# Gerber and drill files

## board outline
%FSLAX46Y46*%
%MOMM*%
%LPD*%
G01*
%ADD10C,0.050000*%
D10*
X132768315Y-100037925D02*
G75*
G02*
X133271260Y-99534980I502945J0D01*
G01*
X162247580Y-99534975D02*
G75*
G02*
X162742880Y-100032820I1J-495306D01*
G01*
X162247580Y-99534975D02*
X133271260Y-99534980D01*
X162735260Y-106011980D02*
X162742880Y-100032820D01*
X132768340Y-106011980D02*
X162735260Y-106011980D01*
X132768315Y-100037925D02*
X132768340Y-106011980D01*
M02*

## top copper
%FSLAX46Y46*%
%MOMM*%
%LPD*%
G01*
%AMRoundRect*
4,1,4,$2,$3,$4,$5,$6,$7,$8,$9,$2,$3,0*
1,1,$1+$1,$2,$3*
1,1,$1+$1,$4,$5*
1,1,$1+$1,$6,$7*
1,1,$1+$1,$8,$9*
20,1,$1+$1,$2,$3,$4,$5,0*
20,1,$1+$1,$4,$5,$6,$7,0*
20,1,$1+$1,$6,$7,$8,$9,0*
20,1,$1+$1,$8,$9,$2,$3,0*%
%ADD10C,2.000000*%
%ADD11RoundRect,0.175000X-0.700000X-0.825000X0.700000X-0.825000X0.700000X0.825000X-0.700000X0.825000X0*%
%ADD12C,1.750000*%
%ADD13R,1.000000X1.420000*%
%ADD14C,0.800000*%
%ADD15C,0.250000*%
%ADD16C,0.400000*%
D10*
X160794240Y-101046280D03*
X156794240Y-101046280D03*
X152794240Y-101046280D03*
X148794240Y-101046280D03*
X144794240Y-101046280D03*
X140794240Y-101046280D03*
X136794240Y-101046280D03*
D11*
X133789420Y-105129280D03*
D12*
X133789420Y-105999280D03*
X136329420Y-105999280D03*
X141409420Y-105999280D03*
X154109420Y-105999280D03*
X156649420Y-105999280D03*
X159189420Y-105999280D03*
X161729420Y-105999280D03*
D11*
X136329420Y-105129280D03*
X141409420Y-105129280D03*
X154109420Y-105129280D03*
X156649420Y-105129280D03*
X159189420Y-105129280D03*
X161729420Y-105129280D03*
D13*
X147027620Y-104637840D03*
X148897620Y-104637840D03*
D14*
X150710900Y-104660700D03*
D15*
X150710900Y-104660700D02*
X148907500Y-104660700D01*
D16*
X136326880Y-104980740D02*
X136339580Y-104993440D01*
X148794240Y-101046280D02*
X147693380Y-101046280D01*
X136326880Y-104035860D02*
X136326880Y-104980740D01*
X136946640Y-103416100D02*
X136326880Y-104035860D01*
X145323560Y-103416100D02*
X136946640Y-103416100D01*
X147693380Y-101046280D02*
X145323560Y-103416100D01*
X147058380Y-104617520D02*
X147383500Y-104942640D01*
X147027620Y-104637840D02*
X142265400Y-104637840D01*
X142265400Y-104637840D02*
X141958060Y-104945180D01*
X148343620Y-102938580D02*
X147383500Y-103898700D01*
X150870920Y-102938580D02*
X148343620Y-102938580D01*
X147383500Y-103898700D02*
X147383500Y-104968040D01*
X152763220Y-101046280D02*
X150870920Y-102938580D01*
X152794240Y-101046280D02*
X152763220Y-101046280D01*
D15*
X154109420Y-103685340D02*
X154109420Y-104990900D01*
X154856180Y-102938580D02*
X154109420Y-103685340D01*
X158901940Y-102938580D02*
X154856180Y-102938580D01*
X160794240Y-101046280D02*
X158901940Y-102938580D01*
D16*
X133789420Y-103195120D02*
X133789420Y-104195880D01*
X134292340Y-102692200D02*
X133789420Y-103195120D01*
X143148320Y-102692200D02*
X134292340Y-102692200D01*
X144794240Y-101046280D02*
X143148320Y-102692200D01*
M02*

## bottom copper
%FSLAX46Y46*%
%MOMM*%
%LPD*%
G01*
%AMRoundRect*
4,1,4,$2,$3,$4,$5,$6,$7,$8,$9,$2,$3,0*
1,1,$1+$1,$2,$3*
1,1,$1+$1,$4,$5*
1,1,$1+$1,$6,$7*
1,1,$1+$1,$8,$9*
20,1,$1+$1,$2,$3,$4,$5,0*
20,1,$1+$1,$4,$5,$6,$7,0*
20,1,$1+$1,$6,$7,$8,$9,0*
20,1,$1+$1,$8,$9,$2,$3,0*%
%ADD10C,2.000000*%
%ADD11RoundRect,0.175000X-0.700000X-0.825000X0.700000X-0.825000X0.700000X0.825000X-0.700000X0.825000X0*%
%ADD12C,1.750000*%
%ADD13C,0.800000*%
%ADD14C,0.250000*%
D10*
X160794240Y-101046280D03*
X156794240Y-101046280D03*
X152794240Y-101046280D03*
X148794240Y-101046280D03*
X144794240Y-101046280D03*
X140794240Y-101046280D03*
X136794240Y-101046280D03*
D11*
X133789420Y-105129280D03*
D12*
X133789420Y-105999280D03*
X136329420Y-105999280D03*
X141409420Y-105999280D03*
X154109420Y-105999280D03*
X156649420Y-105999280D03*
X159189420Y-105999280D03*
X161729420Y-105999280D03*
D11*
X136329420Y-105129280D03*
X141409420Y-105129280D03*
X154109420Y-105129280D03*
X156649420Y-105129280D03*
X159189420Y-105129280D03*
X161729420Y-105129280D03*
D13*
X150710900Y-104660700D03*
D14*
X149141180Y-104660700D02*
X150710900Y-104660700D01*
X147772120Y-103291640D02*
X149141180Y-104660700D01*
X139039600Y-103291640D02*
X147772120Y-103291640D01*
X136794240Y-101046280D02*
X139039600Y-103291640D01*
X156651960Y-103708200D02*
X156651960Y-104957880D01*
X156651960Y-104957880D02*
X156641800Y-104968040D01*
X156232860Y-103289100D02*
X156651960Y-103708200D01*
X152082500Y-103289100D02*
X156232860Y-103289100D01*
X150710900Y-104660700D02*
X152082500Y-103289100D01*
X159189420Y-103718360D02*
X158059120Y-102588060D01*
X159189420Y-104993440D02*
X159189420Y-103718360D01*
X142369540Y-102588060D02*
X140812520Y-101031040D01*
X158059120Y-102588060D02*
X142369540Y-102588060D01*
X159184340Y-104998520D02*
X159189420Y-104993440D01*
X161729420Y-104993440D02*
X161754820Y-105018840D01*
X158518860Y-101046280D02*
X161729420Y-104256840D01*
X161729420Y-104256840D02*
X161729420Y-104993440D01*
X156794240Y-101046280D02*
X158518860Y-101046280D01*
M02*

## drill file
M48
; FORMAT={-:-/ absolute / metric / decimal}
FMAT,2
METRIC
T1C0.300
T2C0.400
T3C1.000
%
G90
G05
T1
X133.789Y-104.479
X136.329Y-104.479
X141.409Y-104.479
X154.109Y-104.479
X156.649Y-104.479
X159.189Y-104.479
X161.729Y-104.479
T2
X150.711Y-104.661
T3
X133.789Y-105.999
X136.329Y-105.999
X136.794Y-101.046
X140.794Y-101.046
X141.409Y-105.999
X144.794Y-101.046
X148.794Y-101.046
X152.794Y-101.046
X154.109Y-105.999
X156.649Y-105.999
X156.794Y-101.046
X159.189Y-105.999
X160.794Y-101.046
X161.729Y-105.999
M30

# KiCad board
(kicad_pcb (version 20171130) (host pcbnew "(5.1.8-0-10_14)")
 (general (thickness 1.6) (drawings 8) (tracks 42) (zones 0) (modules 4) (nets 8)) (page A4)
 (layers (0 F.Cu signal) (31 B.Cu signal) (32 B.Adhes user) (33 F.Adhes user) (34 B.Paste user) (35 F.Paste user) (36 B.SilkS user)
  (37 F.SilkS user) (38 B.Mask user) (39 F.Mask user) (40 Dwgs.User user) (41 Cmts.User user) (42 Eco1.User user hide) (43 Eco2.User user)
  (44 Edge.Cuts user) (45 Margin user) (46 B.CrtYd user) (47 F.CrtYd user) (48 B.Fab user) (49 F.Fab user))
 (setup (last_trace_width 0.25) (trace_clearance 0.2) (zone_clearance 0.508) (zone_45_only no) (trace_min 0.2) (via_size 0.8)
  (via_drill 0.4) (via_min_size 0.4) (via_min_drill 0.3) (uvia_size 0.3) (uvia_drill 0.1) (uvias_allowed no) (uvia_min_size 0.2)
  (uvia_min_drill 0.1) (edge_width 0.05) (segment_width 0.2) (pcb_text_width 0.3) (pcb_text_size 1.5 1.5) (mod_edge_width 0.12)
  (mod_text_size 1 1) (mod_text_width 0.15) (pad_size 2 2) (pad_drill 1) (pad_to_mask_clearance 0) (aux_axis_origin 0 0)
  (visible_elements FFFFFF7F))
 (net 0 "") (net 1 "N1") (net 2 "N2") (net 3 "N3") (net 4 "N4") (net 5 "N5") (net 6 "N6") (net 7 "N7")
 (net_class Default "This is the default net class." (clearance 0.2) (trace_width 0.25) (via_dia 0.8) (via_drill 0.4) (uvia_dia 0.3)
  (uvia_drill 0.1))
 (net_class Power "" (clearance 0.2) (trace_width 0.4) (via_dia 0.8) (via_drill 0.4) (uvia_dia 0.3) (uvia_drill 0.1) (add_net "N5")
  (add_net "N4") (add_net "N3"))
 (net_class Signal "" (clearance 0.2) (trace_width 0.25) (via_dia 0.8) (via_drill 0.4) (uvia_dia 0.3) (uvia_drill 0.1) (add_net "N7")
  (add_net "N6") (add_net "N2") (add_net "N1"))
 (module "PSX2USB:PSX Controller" (layer F.Cu) (at 136.79424 101.04628)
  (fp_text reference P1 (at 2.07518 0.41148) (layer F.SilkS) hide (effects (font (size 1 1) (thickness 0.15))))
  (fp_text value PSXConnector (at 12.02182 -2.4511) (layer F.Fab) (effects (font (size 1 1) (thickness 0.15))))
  (pad 7 thru_hole circle (at 24 0) (size 2 2) (drill 1) (layers *.Cu *.Mask) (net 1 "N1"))
  (pad 6 thru_hole circle (at 20 0) (size 2 2) (drill 1) (layers *.Cu *.Mask) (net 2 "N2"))
  (pad 5 thru_hole circle (at 16 0) (size 2 2) (drill 1) (layers *.Cu *.Mask) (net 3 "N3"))
  (pad 4 thru_hole circle (at 12 0) (size 2 2) (drill 1) (layers *.Cu *.Mask) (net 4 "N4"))
  (pad 3 thru_hole circle (at 8 0) (size 2 2) (drill 1) (layers *.Cu *.Mask) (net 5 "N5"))
  (pad 2 thru_hole circle (at 4 0) (size 2 2) (drill 1) (layers *.Cu *.Mask) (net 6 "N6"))
  (pad 1 thru_hole circle (at 0 0) (size 2 2) (drill 1) (layers *.Cu *.Mask) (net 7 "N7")))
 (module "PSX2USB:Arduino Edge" (layer F.Cu) (at 136.32942 105.99928)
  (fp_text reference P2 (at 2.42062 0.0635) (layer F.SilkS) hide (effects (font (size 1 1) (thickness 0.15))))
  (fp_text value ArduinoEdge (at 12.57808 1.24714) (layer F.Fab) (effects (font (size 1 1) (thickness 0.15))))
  (pad 103 thru_hole roundrect (at -2.54 -1.52) (size 1.75 2) (drill 0.3 (offset 0 0.65)) (layers *.Cu *.Mask) (roundrect_rratio 0.1)
   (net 5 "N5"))
  (pad 103 thru_hole circle (at -2.54 0) (size 1.75 1.75) (drill 1) (layers *.Cu *.Mask) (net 5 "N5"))
  (pad 102 thru_hole circle (at 0 0) (size 1.75 1.75) (drill 1) (layers *.Cu *.Mask) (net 4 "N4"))
  (pad 101 thru_hole circle (at 5.08 0) (size 1.75 1.75) (drill 1) (layers *.Cu *.Mask) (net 3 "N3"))
  (pad 15 thru_hole circle (at 17.78 0) (size 1.75 1.75) (drill 1) (layers *.Cu *.Mask) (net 1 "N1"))
  (pad 14 thru_hole circle (at 20.32 0) (size 1.75 1.75) (drill 1) (layers *.Cu *.Mask) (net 7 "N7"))
  (pad 16 thru_hole circle (at 22.86 0) (size 1.75 1.75) (drill 1) (layers *.Cu *.Mask) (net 6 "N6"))
  (pad 10 thru_hole circle (at 25.4 0) (size 1.75 1.75) (drill 1) (layers *.Cu *.Mask) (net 2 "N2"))
  (pad 102 thru_hole roundrect (at 0 -1.52) (size 1.75 2) (drill 0.3 (offset 0 0.65)) (layers *.Cu *.Mask) (roundrect_rratio 0.1)
   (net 4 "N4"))
  (pad 101 thru_hole roundrect (at 5.08 -1.52) (size 1.75 2) (drill 0.3 (offset 0 0.65)) (layers *.Cu *.Mask) (roundrect_rratio 0.1)
   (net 3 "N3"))
  (pad 15 thru_hole roundrect (at 17.78 -1.52) (size 1.75 2) (drill 0.3 (offset 0 0.65)) (layers *.Cu *.Mask) (roundrect_rratio 0.1)
   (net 1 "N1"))
  (pad 14 thru_hole roundrect (at 20.32 -1.52) (size 1.75 2) (drill 0.3 (offset 0 0.65)) (layers *.Cu *.Mask) (roundrect_rratio 0.1)
   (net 7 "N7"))
  (pad 16 thru_hole roundrect (at 22.86 -1.52) (size 1.75 2) (drill 0.3 (offset 0 0.65)) (layers *.Cu *.Mask) (roundrect_rratio 0.1)
   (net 6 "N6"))
  (pad 10 thru_hole roundrect (at 25.4 -1.52) (size 1.75 2) (drill 0.3 (offset 0 0.65)) (layers *.Cu *.Mask) (roundrect_rratio 0.1)
   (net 2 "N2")))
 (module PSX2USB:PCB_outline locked (layer B.Cu) (at 162.74796 99.5299 180)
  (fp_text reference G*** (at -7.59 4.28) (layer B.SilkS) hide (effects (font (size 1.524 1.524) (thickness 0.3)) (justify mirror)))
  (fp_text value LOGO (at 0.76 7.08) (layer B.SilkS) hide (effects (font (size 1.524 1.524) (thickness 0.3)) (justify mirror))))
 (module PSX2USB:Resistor (layer F.Cu) (at 147.96262 104.63784 180)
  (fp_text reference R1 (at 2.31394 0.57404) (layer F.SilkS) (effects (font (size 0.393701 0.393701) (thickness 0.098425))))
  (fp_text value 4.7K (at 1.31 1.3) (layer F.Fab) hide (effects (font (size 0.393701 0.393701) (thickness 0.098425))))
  (pad 2 smd rect (at 0.935 0 180) (size 1 1.42) (layers F.Cu F.Paste F.Mask) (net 3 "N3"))
  (pad 1 smd rect (at -0.935 0 180) (size 1 1.42) (layers F.Cu F.Paste F.Mask) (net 7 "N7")))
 (gr_arc (start 133.27126 100.037925) (end 133.27126 99.53498) (angle -90) (layer Edge.Cuts) (width 0.05))
 (gr_arc (start 162.247581 100.030281) (end 162.74288 100.03282) (angle -90.29382193) (layer Edge.Cuts) (width 0.05))
 (gr_line (start 162.24758 99.534975) (end 133.27126 99.53498) (layer Edge.Cuts) (width 0.05))
 (gr_line (start 162.73526 106.01198) (end 162.74288 100.03282) (layer Edge.Cuts) (width 0.05))
 (gr_line (start 132.76834 106.01198) (end 162.73526 106.01198) (layer Edge.Cuts) (width 0.05))
 (gr_line (start 132.768315 100.037925) (end 132.76834 106.01198) (layer Edge.Cuts) (width 0.05))
 (via (at 150.7109 104.6607) (size 0.8) (drill 0.4) (layers F.Cu B.Cu) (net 7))
 (segment (start 150.7109 104.6607) (end 148.9075 104.6607) (width 0.25) (layer F.Cu) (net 7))
 (segment (start 149.14118 104.6607) (end 150.7109 104.6607) (width 0.25) (layer B.Cu) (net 7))
 (segment (start 147.77212 103.29164) (end 149.14118 104.6607) (width 0.25) (layer B.Cu) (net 7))
 (segment (start 139.0396 103.29164) (end 147.77212 103.29164) (width 0.25) (layer B.Cu) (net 7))
 (segment (start 136.79424 101.04628) (end 139.0396 103.29164) (width 0.25) (layer B.Cu) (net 7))
 (segment (start 156.65196 103.7082) (end 156.65196 104.95788) (width 0.25) (layer B.Cu) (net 7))
 (segment (start 156.65196 104.95788) (end 156.6418 104.96804) (width 0.25) (layer B.Cu) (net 7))
 (segment (start 156.23286 103.2891) (end 156.65196 103.7082) (width 0.25) (layer B.Cu) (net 7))
 (segment (start 152.0825 103.2891) (end 156.23286 103.2891) (width 0.25) (layer B.Cu) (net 7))
 (segment (start 150.7109 104.6607) (end 152.0825 103.2891) (width 0.25) (layer B.Cu) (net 7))
 (segment (start 159.18942 103.71836) (end 158.05912 102.58806) (width 0.25) (layer B.Cu) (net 6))
 (segment (start 159.18942 104.99344) (end 159.18942 103.71836) (width 0.25) (layer B.Cu) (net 6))
 (segment (start 142.36954 102.58806) (end 140.81252 101.03104) (width 0.25) (layer B.Cu) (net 6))
 (segment (start 158.05912 102.58806) (end 142.36954 102.58806) (width 0.25) (layer B.Cu) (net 6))
 (segment (start 159.18434 104.99852) (end 159.18942 104.99344) (width 0.25) (layer B.Cu) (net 6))
 (segment (start 136.32688 104.98074) (end 136.33958 104.99344) (width 0.4) (layer F.Cu) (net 4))
 (segment (start 148.79424 101.04628) (end 147.69338 101.04628) (width 0.4) (layer F.Cu) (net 4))
 (segment (start 136.32688 104.03586) (end 136.32688 104.98074) (width 0.4) (layer F.Cu) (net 4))
 (segment (start 136.94664 103.4161) (end 136.32688 104.03586) (width 0.4) (layer F.Cu) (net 4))
 (segment (start 145.32356 103.4161) (end 136.94664 103.4161) (width 0.4) (layer F.Cu) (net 4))
 (segment (start 147.69338 101.04628) (end 145.32356 103.4161) (width 0.4) (layer F.Cu) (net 4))
 (segment (start 147.05838 104.61752) (end 147.3835 104.94264) (width 0.4) (layer F.Cu) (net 3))
 (segment (start 147.02762 104.63784) (end 142.2654 104.63784) (width 0.4) (layer F.Cu) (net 3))
 (segment (start 142.2654 104.63784) (end 141.95806 104.94518) (width 0.4) (layer F.Cu) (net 3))
 (segment (start 148.34362 102.93858) (end 147.3835 103.8987) (width 0.4) (layer F.Cu) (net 3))
 (segment (start 150.87092 102.93858) (end 148.34362 102.93858) (width 0.4) (layer F.Cu) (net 3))
 (segment (start 147.3835 103.8987) (end 147.3835 104.96804) (width 0.4) (layer F.Cu) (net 3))
 (segment (start 152.76322 101.04628) (end 150.87092 102.93858) (width 0.4) (layer F.Cu) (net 3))
 (segment (start 152.79424 101.04628) (end 152.76322 101.04628) (width 0.4) (layer F.Cu) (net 3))
 (segment (start 161.72942 104.99344) (end 161.75482 105.01884) (width 0.25) (layer B.Cu) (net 2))
 (segment (start 158.51886 101.04628) (end 161.72942 104.25684) (width 0.25) (layer B.Cu) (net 2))
 (segment (start 161.72942 104.25684) (end 161.72942 104.99344) (width 0.25) (layer B.Cu) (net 2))
 (segment (start 156.79424 101.04628) (end 158.51886 101.04628) (width 0.25) (layer B.Cu) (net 2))
 (segment (start 154.10942 103.68534) (end 154.10942 104.9909) (width 0.25) (layer F.Cu) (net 1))
 (segment (start 154.85618 102.93858) (end 154.10942 103.68534) (width 0.25) (layer F.Cu) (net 1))
 (segment (start 158.90194 102.93858) (end 154.85618 102.93858) (width 0.25) (layer F.Cu) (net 1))
 (segment (start 160.79424 101.04628) (end 158.90194 102.93858) (width 0.25) (layer F.Cu) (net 1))
 (segment (start 133.78942 103.19512) (end 133.78942 104.19588) (width 0.4) (layer F.Cu) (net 5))
 (segment (start 134.29234 102.6922) (end 133.78942 103.19512) (width 0.4) (layer F.Cu) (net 5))
 (segment (start 143.14832 102.6922) (end 134.29234 102.6922) (width 0.4) (layer F.Cu) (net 5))
 (segment (start 144.79424 101.04628) (end 143.14832 102.6922) (width 0.4) (layer F.Cu) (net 5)))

